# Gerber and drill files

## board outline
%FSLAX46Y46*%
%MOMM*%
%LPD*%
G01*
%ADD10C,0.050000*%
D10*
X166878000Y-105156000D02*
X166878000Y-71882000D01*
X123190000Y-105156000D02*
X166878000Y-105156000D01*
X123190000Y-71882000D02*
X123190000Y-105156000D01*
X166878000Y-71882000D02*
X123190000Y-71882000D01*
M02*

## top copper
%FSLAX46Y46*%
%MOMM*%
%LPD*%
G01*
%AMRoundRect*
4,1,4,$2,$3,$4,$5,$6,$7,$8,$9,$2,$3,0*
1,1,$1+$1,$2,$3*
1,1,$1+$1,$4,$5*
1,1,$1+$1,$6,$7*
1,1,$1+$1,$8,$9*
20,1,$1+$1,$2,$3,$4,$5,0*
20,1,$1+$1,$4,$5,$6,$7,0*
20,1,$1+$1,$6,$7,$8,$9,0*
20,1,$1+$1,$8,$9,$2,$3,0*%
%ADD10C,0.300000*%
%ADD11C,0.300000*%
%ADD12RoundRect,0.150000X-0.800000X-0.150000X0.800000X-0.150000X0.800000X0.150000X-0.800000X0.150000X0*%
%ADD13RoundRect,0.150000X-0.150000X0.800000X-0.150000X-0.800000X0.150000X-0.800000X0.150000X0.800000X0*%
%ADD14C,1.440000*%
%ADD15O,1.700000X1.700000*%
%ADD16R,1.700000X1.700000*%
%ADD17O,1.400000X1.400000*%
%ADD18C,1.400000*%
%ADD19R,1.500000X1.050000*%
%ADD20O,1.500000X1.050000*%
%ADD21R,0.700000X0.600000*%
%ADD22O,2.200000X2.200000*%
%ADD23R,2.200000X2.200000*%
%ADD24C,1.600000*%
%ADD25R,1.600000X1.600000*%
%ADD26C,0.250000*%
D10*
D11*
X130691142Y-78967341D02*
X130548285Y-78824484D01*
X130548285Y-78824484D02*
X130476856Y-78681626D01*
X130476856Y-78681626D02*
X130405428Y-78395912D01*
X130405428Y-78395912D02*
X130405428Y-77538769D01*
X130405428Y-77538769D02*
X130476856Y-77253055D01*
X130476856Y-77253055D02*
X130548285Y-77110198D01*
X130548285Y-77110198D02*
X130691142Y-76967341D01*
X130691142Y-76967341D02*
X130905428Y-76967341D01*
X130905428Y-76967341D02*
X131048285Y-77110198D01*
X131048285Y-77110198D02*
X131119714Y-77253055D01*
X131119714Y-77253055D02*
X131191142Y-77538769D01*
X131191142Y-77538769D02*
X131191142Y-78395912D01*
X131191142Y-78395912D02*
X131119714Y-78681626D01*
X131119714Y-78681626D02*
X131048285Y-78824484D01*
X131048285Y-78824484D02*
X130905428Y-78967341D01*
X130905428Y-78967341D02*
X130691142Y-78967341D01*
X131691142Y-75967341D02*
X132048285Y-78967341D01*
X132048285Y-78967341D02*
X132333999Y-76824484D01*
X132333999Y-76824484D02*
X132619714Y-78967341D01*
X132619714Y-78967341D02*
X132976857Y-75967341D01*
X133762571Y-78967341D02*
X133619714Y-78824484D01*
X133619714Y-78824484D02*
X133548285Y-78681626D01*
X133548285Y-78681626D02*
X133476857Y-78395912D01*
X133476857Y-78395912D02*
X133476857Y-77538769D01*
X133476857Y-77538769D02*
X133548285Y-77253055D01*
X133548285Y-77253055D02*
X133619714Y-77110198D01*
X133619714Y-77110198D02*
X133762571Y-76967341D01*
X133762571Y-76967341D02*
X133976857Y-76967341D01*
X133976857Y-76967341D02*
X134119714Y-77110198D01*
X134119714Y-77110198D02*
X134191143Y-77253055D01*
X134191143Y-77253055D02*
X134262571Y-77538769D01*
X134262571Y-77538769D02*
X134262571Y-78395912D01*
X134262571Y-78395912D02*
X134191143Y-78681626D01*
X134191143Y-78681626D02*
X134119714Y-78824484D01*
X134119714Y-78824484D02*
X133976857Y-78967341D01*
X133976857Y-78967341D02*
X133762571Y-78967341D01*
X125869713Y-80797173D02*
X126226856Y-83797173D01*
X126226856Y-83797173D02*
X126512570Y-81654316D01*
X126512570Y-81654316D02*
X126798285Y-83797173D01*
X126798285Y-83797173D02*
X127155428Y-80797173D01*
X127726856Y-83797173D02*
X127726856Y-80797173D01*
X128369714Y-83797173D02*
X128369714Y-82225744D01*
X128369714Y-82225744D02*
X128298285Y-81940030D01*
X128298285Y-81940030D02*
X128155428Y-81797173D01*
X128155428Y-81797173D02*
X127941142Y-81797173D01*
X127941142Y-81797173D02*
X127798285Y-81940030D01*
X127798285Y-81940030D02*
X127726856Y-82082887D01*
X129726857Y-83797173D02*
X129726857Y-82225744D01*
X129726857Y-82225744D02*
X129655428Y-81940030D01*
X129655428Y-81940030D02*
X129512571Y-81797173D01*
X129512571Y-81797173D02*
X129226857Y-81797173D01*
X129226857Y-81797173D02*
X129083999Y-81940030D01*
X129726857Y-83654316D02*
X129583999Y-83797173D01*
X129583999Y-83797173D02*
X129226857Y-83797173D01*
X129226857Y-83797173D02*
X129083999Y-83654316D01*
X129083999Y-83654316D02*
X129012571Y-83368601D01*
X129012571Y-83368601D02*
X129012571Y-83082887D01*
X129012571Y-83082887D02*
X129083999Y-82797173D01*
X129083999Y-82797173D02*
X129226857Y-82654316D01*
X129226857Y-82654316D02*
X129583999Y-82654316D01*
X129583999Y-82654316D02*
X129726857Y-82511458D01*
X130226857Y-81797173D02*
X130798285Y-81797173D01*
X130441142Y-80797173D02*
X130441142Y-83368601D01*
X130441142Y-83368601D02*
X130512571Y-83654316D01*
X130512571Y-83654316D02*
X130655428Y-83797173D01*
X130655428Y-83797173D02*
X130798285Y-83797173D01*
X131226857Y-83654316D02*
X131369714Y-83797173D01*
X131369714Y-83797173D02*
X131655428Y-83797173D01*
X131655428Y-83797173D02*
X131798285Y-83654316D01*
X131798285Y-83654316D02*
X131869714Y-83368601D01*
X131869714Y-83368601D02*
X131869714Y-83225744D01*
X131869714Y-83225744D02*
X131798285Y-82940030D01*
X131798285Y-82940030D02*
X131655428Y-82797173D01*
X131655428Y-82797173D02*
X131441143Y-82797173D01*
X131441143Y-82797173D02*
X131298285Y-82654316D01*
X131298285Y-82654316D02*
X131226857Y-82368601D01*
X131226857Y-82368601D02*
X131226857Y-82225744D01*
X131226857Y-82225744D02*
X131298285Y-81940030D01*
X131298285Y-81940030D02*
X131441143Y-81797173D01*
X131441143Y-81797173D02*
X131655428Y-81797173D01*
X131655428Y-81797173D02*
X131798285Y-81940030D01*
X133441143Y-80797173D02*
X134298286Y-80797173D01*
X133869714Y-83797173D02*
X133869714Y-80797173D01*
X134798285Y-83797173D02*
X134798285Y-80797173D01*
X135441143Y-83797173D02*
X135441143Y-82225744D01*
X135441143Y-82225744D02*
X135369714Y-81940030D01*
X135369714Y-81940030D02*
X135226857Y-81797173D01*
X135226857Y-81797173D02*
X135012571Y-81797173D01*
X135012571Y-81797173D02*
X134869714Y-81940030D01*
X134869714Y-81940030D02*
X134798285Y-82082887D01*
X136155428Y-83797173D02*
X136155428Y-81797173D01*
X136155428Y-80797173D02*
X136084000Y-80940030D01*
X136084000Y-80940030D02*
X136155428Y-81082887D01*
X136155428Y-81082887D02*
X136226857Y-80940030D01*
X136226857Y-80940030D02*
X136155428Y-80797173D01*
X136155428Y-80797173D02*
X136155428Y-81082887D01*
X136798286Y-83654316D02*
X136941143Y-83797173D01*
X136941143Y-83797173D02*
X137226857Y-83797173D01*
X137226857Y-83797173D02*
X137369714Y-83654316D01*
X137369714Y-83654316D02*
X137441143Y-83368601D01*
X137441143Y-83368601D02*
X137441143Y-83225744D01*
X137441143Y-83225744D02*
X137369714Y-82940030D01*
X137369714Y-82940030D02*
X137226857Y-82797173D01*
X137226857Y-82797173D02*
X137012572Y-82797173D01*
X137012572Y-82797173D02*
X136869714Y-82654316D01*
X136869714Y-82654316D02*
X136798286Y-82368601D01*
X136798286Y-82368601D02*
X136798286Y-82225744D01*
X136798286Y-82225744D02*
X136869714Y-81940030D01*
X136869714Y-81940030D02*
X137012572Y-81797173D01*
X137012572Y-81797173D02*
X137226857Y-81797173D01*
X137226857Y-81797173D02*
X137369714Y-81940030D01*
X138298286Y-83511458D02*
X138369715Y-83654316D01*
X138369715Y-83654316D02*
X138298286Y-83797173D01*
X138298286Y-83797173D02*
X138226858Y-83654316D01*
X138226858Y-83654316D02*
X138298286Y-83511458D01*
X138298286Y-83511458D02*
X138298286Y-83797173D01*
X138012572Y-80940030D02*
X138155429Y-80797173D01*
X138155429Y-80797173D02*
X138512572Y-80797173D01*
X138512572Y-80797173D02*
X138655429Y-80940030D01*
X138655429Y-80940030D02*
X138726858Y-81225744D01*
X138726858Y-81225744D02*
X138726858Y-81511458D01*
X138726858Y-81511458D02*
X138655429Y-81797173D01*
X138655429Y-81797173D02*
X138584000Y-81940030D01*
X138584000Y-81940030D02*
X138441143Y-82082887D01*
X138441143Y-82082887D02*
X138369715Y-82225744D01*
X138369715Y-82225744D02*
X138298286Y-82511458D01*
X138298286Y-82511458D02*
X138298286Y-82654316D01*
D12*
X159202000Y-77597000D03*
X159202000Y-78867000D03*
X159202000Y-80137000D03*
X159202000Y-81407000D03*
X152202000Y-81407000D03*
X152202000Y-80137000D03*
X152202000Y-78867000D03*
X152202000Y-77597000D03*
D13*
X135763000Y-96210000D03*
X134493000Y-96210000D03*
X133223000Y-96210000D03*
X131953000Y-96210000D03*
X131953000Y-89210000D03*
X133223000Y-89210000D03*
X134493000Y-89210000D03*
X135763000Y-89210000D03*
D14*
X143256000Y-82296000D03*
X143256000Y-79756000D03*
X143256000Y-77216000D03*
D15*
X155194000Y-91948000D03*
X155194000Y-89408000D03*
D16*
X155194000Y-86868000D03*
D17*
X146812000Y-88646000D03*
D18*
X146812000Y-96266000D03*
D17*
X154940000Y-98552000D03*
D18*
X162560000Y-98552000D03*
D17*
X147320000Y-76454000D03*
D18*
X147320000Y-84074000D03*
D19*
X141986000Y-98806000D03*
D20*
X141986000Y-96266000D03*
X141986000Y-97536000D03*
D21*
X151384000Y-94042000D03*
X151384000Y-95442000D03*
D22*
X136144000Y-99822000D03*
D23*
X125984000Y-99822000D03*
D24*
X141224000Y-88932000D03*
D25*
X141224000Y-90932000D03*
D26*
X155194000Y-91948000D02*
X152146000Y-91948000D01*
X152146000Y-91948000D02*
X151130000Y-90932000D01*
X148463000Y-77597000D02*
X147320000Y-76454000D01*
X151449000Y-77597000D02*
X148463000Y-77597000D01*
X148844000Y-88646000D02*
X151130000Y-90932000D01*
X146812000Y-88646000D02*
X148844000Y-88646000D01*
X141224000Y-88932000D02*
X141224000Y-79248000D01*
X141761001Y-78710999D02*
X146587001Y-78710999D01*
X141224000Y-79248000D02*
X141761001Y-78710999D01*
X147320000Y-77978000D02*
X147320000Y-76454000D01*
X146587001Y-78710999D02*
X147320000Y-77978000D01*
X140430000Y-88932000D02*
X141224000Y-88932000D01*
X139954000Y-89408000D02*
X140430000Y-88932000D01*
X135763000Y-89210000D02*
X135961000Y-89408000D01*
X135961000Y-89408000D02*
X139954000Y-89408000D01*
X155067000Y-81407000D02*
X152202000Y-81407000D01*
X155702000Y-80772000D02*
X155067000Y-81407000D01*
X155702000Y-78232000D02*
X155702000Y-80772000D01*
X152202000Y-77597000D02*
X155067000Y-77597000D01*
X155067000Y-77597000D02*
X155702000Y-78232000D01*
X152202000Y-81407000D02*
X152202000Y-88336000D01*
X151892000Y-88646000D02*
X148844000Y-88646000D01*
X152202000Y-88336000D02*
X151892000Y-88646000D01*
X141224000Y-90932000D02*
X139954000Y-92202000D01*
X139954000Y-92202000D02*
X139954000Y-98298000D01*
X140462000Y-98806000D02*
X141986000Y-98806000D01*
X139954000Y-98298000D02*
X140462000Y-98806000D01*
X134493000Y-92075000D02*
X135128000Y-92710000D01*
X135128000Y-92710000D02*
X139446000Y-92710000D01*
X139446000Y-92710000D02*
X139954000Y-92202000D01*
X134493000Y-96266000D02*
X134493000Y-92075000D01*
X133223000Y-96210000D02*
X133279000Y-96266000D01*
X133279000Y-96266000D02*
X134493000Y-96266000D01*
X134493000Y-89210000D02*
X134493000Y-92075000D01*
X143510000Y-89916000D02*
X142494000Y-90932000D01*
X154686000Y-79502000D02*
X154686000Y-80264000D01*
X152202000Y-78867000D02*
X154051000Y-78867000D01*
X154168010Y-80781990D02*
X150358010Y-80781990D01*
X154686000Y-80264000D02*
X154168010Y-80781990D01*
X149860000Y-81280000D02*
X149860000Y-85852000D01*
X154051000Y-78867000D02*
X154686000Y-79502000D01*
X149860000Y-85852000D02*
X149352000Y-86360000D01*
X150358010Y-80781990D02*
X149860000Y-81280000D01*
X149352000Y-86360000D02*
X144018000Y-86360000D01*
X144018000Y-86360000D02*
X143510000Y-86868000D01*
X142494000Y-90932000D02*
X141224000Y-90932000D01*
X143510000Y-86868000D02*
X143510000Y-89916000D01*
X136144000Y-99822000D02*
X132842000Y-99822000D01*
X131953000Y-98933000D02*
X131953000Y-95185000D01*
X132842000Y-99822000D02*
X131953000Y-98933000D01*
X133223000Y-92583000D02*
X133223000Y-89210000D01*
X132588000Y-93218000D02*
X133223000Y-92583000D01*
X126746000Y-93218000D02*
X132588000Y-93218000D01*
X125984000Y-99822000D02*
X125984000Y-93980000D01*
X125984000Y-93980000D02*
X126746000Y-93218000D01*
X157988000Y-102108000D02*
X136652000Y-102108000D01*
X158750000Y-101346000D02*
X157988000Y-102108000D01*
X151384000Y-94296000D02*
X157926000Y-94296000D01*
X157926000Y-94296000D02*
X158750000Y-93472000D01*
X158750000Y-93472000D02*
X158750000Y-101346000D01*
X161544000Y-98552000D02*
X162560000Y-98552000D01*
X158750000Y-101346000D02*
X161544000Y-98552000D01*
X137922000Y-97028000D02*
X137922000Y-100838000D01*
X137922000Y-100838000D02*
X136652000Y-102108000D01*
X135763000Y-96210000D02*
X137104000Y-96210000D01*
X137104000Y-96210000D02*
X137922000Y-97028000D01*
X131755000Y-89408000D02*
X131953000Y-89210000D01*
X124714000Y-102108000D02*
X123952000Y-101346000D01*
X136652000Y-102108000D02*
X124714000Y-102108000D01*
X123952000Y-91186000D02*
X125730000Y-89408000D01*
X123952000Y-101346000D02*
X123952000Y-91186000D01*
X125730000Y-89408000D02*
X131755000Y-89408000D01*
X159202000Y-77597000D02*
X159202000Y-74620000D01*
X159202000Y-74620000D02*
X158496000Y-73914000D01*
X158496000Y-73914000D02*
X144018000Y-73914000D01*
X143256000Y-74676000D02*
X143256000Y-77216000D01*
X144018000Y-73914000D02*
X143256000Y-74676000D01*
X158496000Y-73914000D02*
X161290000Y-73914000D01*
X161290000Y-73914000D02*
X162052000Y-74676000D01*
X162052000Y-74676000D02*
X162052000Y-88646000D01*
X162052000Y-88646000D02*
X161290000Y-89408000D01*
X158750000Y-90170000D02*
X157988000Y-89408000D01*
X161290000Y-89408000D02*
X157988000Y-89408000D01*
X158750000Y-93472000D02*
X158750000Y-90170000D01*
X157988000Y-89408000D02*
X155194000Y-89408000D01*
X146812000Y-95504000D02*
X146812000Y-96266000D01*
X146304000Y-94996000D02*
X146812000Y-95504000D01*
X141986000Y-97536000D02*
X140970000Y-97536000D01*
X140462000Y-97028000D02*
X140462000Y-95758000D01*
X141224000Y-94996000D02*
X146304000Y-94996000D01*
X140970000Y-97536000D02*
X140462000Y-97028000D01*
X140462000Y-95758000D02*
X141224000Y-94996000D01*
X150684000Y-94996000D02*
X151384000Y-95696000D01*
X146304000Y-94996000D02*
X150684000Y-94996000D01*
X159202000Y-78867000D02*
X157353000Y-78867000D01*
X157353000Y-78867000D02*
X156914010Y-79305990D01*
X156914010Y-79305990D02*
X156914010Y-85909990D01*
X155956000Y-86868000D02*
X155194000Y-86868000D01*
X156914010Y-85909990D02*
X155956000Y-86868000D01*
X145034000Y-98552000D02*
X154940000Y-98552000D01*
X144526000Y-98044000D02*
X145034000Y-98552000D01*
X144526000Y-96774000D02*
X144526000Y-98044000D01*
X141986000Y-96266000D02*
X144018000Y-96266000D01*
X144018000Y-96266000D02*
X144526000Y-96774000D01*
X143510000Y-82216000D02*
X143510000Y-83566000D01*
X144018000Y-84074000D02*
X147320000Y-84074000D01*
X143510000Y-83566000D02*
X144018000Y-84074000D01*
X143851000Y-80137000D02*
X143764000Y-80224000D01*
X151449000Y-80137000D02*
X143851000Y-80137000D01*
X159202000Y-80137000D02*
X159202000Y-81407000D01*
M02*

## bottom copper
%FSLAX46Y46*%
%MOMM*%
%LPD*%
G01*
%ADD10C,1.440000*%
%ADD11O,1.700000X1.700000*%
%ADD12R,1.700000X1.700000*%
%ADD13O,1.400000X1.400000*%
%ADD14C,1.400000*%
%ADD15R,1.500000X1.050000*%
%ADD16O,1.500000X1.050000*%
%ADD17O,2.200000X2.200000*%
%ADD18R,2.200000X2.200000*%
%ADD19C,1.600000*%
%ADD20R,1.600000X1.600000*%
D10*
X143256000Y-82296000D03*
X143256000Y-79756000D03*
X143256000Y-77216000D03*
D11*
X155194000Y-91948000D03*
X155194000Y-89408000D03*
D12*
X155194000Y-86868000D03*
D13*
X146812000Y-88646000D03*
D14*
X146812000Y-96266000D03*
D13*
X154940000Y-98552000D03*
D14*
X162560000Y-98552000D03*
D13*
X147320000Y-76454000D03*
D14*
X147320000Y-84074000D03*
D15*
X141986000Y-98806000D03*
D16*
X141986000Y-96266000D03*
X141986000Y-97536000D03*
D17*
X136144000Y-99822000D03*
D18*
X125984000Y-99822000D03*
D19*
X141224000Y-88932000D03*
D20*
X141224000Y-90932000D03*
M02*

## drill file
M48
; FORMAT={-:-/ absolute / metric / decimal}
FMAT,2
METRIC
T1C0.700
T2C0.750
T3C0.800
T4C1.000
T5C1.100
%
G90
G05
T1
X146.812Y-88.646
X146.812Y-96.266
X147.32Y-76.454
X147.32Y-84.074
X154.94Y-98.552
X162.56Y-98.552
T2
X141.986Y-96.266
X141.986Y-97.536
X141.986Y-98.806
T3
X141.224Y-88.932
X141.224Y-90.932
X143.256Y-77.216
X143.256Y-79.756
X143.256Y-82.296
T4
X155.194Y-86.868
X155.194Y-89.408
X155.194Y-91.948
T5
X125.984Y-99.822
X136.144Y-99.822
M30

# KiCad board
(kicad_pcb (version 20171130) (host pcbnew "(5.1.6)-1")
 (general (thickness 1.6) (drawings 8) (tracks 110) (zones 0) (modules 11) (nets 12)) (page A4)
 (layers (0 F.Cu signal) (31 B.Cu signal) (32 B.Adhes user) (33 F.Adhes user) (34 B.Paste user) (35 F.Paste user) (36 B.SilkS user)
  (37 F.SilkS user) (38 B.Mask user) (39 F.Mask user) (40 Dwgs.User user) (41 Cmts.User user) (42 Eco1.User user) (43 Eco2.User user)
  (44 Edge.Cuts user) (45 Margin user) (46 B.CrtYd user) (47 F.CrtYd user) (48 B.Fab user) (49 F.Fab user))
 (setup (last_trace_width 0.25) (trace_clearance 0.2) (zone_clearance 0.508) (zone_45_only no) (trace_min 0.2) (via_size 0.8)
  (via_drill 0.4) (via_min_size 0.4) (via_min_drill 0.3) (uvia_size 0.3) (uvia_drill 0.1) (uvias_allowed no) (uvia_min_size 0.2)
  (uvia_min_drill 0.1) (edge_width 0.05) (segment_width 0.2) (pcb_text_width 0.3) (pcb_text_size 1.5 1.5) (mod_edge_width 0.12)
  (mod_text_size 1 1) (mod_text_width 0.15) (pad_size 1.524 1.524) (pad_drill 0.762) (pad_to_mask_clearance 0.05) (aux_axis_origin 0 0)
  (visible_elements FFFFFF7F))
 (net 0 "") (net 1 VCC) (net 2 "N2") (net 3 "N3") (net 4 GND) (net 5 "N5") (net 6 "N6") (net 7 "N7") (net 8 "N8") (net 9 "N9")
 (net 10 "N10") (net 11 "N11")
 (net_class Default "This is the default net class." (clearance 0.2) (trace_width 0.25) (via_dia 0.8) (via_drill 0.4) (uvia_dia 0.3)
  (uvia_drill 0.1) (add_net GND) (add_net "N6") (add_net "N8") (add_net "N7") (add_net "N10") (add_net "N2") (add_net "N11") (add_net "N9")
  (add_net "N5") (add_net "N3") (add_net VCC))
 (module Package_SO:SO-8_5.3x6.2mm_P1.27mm (layer F.Cu) (at 155.702 79.502)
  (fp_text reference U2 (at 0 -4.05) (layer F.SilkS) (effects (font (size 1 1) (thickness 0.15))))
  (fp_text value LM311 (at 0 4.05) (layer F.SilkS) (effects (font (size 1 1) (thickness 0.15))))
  (pad 8 smd roundrect (at 3.5 -1.905) (size 1.9 0.6) (layers F.Cu F.Paste F.Mask) (roundrect_rratio 0.25) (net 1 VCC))
  (pad 7 smd roundrect (at 3.5 -0.635) (size 1.9 0.6) (layers F.Cu F.Paste F.Mask) (roundrect_rratio 0.25) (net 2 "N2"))
  (pad 6 smd roundrect (at 3.5 0.635) (size 1.9 0.6) (layers F.Cu F.Paste F.Mask) (roundrect_rratio 0.25) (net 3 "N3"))
  (pad 5 smd roundrect (at 3.5 1.905) (size 1.9 0.6) (layers F.Cu F.Paste F.Mask) (roundrect_rratio 0.25) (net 3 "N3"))
  (pad 4 smd roundrect (at -3.5 1.905) (size 1.9 0.6) (layers F.Cu F.Paste F.Mask) (roundrect_rratio 0.25) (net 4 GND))
  (pad 3 smd roundrect (at -3.5 0.635) (size 1.9 0.6) (layers F.Cu F.Paste F.Mask) (roundrect_rratio 0.25) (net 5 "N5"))
  (pad 2 smd roundrect (at -3.5 -0.635) (size 1.9 0.6) (layers F.Cu F.Paste F.Mask) (roundrect_rratio 0.25) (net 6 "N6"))
  (pad 1 smd roundrect (at -3.5 -1.905) (size 1.9 0.6) (layers F.Cu F.Paste F.Mask) (roundrect_rratio 0.25) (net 4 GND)))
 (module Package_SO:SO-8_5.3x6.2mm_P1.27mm (layer F.Cu) (at 133.858 92.71 270)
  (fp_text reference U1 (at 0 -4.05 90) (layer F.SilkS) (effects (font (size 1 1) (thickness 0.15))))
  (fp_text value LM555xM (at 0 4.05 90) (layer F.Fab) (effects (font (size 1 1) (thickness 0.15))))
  (pad 8 smd roundrect (at 3.5 -1.905 270) (size 1.9 0.6) (layers F.Cu F.Paste F.Mask) (roundrect_rratio 0.25) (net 1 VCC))
  (pad 7 smd roundrect (at 3.5 -0.635 270) (size 1.9 0.6) (layers F.Cu F.Paste F.Mask) (roundrect_rratio 0.25) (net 6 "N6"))
  (pad 6 smd roundrect (at 3.5 0.635 270) (size 1.9 0.6) (layers F.Cu F.Paste F.Mask) (roundrect_rratio 0.25) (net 6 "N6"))
  (pad 5 smd roundrect (at 3.5 1.905 270) (size 1.9 0.6) (layers F.Cu F.Paste F.Mask) (roundrect_rratio 0.25) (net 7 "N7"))
  (pad 4 smd roundrect (at -3.5 1.905 270) (size 1.9 0.6) (layers F.Cu F.Paste F.Mask) (roundrect_rratio 0.25) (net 1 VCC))
  (pad 3 smd roundrect (at -3.5 0.635 270) (size 1.9 0.6) (layers F.Cu F.Paste F.Mask) (roundrect_rratio 0.25) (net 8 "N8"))
  (pad 2 smd roundrect (at -3.5 -0.635 270) (size 1.9 0.6) (layers F.Cu F.Paste F.Mask) (roundrect_rratio 0.25) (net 6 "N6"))
  (pad 1 smd roundrect (at -3.5 -1.905 270) (size 1.9 0.6) (layers F.Cu F.Paste F.Mask) (roundrect_rratio 0.25) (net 4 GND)))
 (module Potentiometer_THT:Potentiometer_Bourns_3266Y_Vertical (layer F.Cu) (at 143.256 77.216 90)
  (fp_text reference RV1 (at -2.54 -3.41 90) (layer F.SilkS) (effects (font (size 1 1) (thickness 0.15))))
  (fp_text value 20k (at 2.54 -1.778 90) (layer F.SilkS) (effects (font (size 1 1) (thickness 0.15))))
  (pad 3 thru_hole circle (at -5.08 0 90) (size 1.44 1.44) (drill 0.8) (layers *.Cu *.Mask) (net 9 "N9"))
  (pad 2 thru_hole circle (at -2.54 0 90) (size 1.44 1.44) (drill 0.8) (layers *.Cu *.Mask) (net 5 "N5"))
  (pad 1 thru_hole circle (at 0 0 90) (size 1.44 1.44) (drill 0.8) (layers *.Cu *.Mask) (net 1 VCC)))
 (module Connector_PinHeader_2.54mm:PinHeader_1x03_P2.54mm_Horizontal (layer F.Cu) (at 155.194 86.868)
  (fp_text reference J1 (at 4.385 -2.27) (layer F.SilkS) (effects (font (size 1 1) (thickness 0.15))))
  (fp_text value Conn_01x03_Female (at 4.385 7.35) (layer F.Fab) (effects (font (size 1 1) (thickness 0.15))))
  (pad 3 thru_hole oval (at 0 5.08) (size 1.7 1.7) (drill 1) (layers *.Cu *.Mask) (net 4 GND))
  (pad 2 thru_hole oval (at 0 2.54) (size 1.7 1.7) (drill 1) (layers *.Cu *.Mask) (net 1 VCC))
  (pad 1 thru_hole rect (at 0 0) (size 1.7 1.7) (drill 1) (layers *.Cu *.Mask) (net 2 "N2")))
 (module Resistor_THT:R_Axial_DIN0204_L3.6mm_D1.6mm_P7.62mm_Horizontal (layer F.Cu) (at 146.812 96.266 90)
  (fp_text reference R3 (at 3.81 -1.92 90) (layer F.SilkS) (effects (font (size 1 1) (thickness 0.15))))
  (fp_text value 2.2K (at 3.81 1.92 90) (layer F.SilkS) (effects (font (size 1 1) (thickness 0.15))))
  (pad 2 thru_hole oval (at 7.62 0 90) (size 1.4 1.4) (drill 0.7) (layers *.Cu *.Mask) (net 4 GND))
  (pad 1 thru_hole circle (at 0 0 90) (size 1.4 1.4) (drill 0.7) (layers *.Cu *.Mask) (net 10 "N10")))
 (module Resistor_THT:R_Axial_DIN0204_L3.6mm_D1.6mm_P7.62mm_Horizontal (layer F.Cu) (at 162.56 98.552 180)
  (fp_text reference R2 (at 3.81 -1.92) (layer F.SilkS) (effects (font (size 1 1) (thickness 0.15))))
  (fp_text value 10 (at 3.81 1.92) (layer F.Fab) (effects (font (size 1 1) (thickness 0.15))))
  (pad 2 thru_hole oval (at 7.62 0 180) (size 1.4 1.4) (drill 0.7) (layers *.Cu *.Mask) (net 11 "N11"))
  (pad 1 thru_hole circle (at 0 0 180) (size 1.4 1.4) (drill 0.7) (layers *.Cu *.Mask) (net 1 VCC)))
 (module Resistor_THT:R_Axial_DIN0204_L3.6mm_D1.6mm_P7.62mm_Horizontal (layer F.Cu) (at 147.32 84.074 90)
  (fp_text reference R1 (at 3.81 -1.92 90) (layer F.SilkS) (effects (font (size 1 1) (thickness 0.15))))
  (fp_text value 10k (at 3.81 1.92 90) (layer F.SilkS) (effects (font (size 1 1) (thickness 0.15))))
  (pad 2 thru_hole oval (at 7.62 0 90) (size 1.4 1.4) (drill 0.7) (layers *.Cu *.Mask) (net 4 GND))
  (pad 1 thru_hole circle (at 0 0 90) (size 1.4 1.4) (drill 0.7) (layers *.Cu *.Mask) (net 9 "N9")))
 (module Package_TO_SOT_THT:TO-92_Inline (layer F.Cu) (at 141.986 98.806 90)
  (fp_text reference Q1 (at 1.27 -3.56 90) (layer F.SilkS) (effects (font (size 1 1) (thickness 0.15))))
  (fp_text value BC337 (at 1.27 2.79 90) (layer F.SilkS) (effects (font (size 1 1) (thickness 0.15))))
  (pad 1 thru_hole rect (at 0 0 90) (size 1.05 1.5) (drill 0.75) (layers *.Cu *.Mask) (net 6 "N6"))
  (pad 3 thru_hole oval (at 2.54 0 90) (size 1.05 1.5) (drill 0.75) (layers *.Cu *.Mask) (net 11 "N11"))
  (pad 2 thru_hole oval (at 1.27 0 90) (size 1.05 1.5) (drill 0.75) (layers *.Cu *.Mask) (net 10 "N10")))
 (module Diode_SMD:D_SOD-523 (layer F.Cu) (at 151.384 94.742 270)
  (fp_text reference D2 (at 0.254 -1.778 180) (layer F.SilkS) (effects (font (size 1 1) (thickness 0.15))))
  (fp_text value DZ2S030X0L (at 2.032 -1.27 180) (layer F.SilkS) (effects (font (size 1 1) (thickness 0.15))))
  (pad 1 smd rect (at -0.7 0 90) (size 0.6 0.7) (layers F.Cu F.Paste F.Mask) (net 1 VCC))
  (pad 2 smd rect (at 0.7 0 90) (size 0.6 0.7) (layers F.Cu F.Paste F.Mask) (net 10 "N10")))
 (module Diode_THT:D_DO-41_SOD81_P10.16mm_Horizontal (layer F.Cu) (at 125.984 99.822)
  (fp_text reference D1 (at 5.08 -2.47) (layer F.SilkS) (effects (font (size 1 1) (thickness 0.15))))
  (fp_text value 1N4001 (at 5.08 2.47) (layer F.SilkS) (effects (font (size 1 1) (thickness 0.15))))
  (pad 2 thru_hole oval (at 10.16 0) (size 2.2 2.2) (drill 1.1) (layers *.Cu *.Mask) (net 7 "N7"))
  (pad 1 thru_hole rect (at 0 0) (size 2.2 2.2) (drill 1.1) (layers *.Cu *.Mask) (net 8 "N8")))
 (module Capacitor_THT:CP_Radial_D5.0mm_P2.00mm (layer F.Cu) (at 141.224 90.932 90)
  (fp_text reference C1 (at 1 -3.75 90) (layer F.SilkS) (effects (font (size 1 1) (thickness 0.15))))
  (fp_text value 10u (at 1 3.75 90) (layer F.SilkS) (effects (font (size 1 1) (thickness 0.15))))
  (pad 2 thru_hole circle (at 2 0 90) (size 1.6 1.6) (drill 0.8) (layers *.Cu *.Mask) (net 4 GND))
  (pad 1 thru_hole rect (at 0 0 90) (size 1.6 1.6) (drill 0.8) (layers *.Cu *.Mask) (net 6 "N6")))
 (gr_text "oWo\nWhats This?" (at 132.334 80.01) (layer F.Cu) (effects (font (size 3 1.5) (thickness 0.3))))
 (gr_line (start 166.878 105.156) (end 166.878 71.882) (layer Edge.Cuts) (width 0.05))
 (gr_line (start 123.19 105.156) (end 166.878 105.156) (layer Edge.Cuts) (width 0.05))
 (gr_line (start 123.19 71.882) (end 123.19 105.156) (layer Edge.Cuts) (width 0.05))
 (gr_line (start 166.878 71.882) (end 123.19 71.882) (layer Edge.Cuts) (width 0.05))
 (segment (start 155.194 91.948) (end 152.146 91.948) (width 0.25) (layer F.Cu) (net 4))
 (segment (start 152.146 91.948) (end 151.13 90.932) (width 0.25) (layer F.Cu) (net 4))
 (segment (start 148.463 77.597) (end 147.32 76.454) (width 0.25) (layer F.Cu) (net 4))
 (segment (start 151.449 77.597) (end 148.463 77.597) (width 0.25) (layer F.Cu) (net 4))
 (segment (start 148.844 88.646) (end 151.13 90.932) (width 0.25) (layer F.Cu) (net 4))
 (segment (start 146.812 88.646) (end 148.844 88.646) (width 0.25) (layer F.Cu) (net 4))
 (segment (start 141.224 88.932) (end 141.224 79.248) (width 0.25) (layer F.Cu) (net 4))
 (segment (start 141.761001 78.710999) (end 146.587001 78.710999) (width 0.25) (layer F.Cu) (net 4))
 (segment (start 141.224 79.248) (end 141.761001 78.710999) (width 0.25) (layer F.Cu) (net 4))
 (segment (start 147.32 77.978) (end 147.32 76.454) (width 0.25) (layer F.Cu) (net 4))
 (segment (start 146.587001 78.710999) (end 147.32 77.978) (width 0.25) (layer F.Cu) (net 4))
 (segment (start 140.43 88.932) (end 141.224 88.932) (width 0.25) (layer F.Cu) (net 4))
 (segment (start 139.954 89.408) (end 140.43 88.932) (width 0.25) (layer F.Cu) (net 4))
 (segment (start 135.763 89.21) (end 135.961 89.408) (width 0.25) (layer F.Cu) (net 4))
 (segment (start 135.961 89.408) (end 139.954 89.408) (width 0.25) (layer F.Cu) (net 4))
 (segment (start 155.067 81.407) (end 152.202 81.407) (width 0.25) (layer F.Cu) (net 4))
 (segment (start 155.702 80.772) (end 155.067 81.407) (width 0.25) (layer F.Cu) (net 4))
 (segment (start 155.702 78.232) (end 155.702 80.772) (width 0.25) (layer F.Cu) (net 4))
 (segment (start 152.202 77.597) (end 155.067 77.597) (width 0.25) (layer F.Cu) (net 4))
 (segment (start 155.067 77.597) (end 155.702 78.232) (width 0.25) (layer F.Cu) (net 4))
 (segment (start 152.202 81.407) (end 152.202 88.336) (width 0.25) (layer F.Cu) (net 4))
 (segment (start 151.892 88.646) (end 148.844 88.646) (width 0.25) (layer F.Cu) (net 4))
 (segment (start 152.202 88.336) (end 151.892 88.646) (width 0.25) (layer F.Cu) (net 4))
 (segment (start 141.224 90.932) (end 139.954 92.202) (width 0.25) (layer F.Cu) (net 6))
 (segment (start 139.954 92.202) (end 139.954 98.298) (width 0.25) (layer F.Cu) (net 6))
 (segment (start 140.462 98.806) (end 141.986 98.806) (width 0.25) (layer F.Cu) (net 6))
 (segment (start 139.954 98.298) (end 140.462 98.806) (width 0.25) (layer F.Cu) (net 6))
 (segment (start 134.493 92.075) (end 135.128 92.71) (width 0.25) (layer F.Cu) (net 6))
 (segment (start 135.128 92.71) (end 139.446 92.71) (width 0.25) (layer F.Cu) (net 6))
 (segment (start 139.446 92.71) (end 139.954 92.202) (width 0.25) (layer F.Cu) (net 6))
 (segment (start 134.493 96.266) (end 134.493 92.075) (width 0.25) (layer F.Cu) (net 6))
 (segment (start 133.223 96.21) (end 133.279 96.266) (width 0.25) (layer F.Cu) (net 6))
 (segment (start 133.279 96.266) (end 134.493 96.266) (width 0.25) (layer F.Cu) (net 6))
 (segment (start 134.493 89.21) (end 134.493 92.075) (width 0.25) (layer F.Cu) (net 6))
 (segment (start 143.51 89.916) (end 142.494 90.932) (width 0.25) (layer F.Cu) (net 6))
 (segment (start 154.686 79.502) (end 154.686 80.264) (width 0.25) (layer F.Cu) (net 6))
 (segment (start 152.202 78.867) (end 154.051 78.867) (width 0.25) (layer F.Cu) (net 6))
 (segment (start 154.16801 80.78199) (end 150.35801 80.78199) (width 0.25) (layer F.Cu) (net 6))
 (segment (start 154.686 80.264) (end 154.16801 80.78199) (width 0.25) (layer F.Cu) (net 6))
 (segment (start 149.86 81.28) (end 149.86 85.852) (width 0.25) (layer F.Cu) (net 6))
 (segment (start 154.051 78.867) (end 154.686 79.502) (width 0.25) (layer F.Cu) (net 6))
 (segment (start 149.86 85.852) (end 149.352 86.36) (width 0.25) (layer F.Cu) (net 6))
 (segment (start 150.35801 80.78199) (end 149.86 81.28) (width 0.25) (layer F.Cu) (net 6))
 (segment (start 149.352 86.36) (end 144.018 86.36) (width 0.25) (layer F.Cu) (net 6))
 (segment (start 144.018 86.36) (end 143.51 86.868) (width 0.25) (layer F.Cu) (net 6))
 (segment (start 142.494 90.932) (end 141.224 90.932) (width 0.25) (layer F.Cu) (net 6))
 (segment (start 143.51 86.868) (end 143.51 89.916) (width 0.25) (layer F.Cu) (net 6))
 (segment (start 136.144 99.822) (end 132.842 99.822) (width 0.25) (layer F.Cu) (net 7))
 (segment (start 131.953 98.933) (end 131.953 95.185) (width 0.25) (layer F.Cu) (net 7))
 (segment (start 132.842 99.822) (end 131.953 98.933) (width 0.25) (layer F.Cu) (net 7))
 (segment (start 133.223 92.583) (end 133.223 89.21) (width 0.25) (layer F.Cu) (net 8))
 (segment (start 132.588 93.218) (end 133.223 92.583) (width 0.25) (layer F.Cu) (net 8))
 (segment (start 126.746 93.218) (end 132.588 93.218) (width 0.25) (layer F.Cu) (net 8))
 (segment (start 125.984 99.822) (end 125.984 93.98) (width 0.25) (layer F.Cu) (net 8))
 (segment (start 125.984 93.98) (end 126.746 93.218) (width 0.25) (layer F.Cu) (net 8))
 (segment (start 157.988 102.108) (end 136.652 102.108) (width 0.25) (layer F.Cu) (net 1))
 (segment (start 158.75 101.346) (end 157.988 102.108) (width 0.25) (layer F.Cu) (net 1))
 (segment (start 151.384 94.296) (end 157.926 94.296) (width 0.25) (layer F.Cu) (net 1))
 (segment (start 157.926 94.296) (end 158.75 93.472) (width 0.25) (layer F.Cu) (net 1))
 (segment (start 158.75 93.472) (end 158.75 101.346) (width 0.25) (layer F.Cu) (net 1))
 (segment (start 161.544 98.552) (end 162.56 98.552) (width 0.25) (layer F.Cu) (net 1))
 (segment (start 158.75 101.346) (end 161.544 98.552) (width 0.25) (layer F.Cu) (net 1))
 (segment (start 137.922 97.028) (end 137.922 100.838) (width 0.25) (layer F.Cu) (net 1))
 (segment (start 137.922 100.838) (end 136.652 102.108) (width 0.25) (layer F.Cu) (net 1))
 (segment (start 135.763 96.21) (end 137.104 96.21) (width 0.25) (layer F.Cu) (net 1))
 (segment (start 137.104 96.21) (end 137.922 97.028) (width 0.25) (layer F.Cu) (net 1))
 (segment (start 131.755 89.408) (end 131.953 89.21) (width 0.25) (layer F.Cu) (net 1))
 (segment (start 124.714 102.108) (end 123.952 101.346) (width 0.25) (layer F.Cu) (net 1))
 (segment (start 136.652 102.108) (end 124.714 102.108) (width 0.25) (layer F.Cu) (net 1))
 (segment (start 123.952 91.186) (end 125.73 89.408) (width 0.25) (layer F.Cu) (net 1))
 (segment (start 123.952 101.346) (end 123.952 91.186) (width 0.25) (layer F.Cu) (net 1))
 (segment (start 125.73 89.408) (end 131.755 89.408) (width 0.25) (layer F.Cu) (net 1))
 (segment (start 159.202 77.597) (end 159.202 74.62) (width 0.25) (layer F.Cu) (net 1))
 (segment (start 159.202 74.62) (end 158.496 73.914) (width 0.25) (layer F.Cu) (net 1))
 (segment (start 158.496 73.914) (end 144.018 73.914) (width 0.25) (layer F.Cu) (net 1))
 (segment (start 143.256 74.676) (end 143.256 77.216) (width 0.25) (layer F.Cu) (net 1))
 (segment (start 144.018 73.914) (end 143.256 74.676) (width 0.25) (layer F.Cu) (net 1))
 (segment (start 158.496 73.914) (end 161.29 73.914) (width 0.25) (layer F.Cu) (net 1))
 (segment (start 161.29 73.914) (end 162.052 74.676) (width 0.25) (layer F.Cu) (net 1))
 (segment (start 162.052 74.676) (end 162.052 88.646) (width 0.25) (layer F.Cu) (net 1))
 (segment (start 162.052 88.646) (end 161.29 89.408) (width 0.25) (layer F.Cu) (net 1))
 (segment (start 158.75 90.17) (end 157.988 89.408) (width 0.25) (layer F.Cu) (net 1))
 (segment (start 161.29 89.408) (end 157.988 89.408) (width 0.25) (layer F.Cu) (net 1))
 (segment (start 158.75 93.472) (end 158.75 90.17) (width 0.25) (layer F.Cu) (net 1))
 (segment (start 157.988 89.408) (end 155.194 89.408) (width 0.25) (layer F.Cu) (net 1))
 (segment (start 146.812 95.504) (end 146.812 96.266) (width 0.25) (layer F.Cu) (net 10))
 (segment (start 146.304 94.996) (end 146.812 95.504) (width 0.25) (layer F.Cu) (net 10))
 (segment (start 141.986 97.536) (end 140.97 97.536) (width 0.25) (layer F.Cu) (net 10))
 (segment (start 140.462 97.028) (end 140.462 95.758) (width 0.25) (layer F.Cu) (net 10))
 (segment (start 141.224 94.996) (end 146.304 94.996) (width 0.25) (layer F.Cu) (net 10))
 (segment (start 140.97 97.536) (end 140.462 97.028) (width 0.25) (layer F.Cu) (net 10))
 (segment (start 140.462 95.758) (end 141.224 94.996) (width 0.25) (layer F.Cu) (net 10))
 (segment (start 150.684 94.996) (end 151.384 95.696) (width 0.25) (layer F.Cu) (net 10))
 (segment (start 146.304 94.996) (end 150.684 94.996) (width 0.25) (layer F.Cu) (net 10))
 (segment (start 159.202 78.867) (end 157.353 78.867) (width 0.25) (layer F.Cu) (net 2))
 (segment (start 157.353 78.867) (end 156.91401 79.30599) (width 0.25) (layer F.Cu) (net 2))
 (segment (start 156.91401 79.30599) (end 156.91401 85.90999) (width 0.25) (layer F.Cu) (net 2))
 (segment (start 155.956 86.868) (end 155.194 86.868) (width 0.25) (layer F.Cu) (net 2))
 (segment (start 156.91401 85.90999) (end 155.956 86.868) (width 0.25) (layer F.Cu) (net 2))
 (segment (start 145.034 98.552) (end 154.94 98.552) (width 0.25) (layer F.Cu) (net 11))
 (segment (start 144.526 98.044) (end 145.034 98.552) (width 0.25) (layer F.Cu) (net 11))
 (segment (start 144.526 96.774) (end 144.526 98.044) (width 0.25) (layer F.Cu) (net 11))
 (segment (start 141.986 96.266) (end 144.018 96.266) (width 0.25) (layer F.Cu) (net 11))
 (segment (start 144.018 96.266) (end 144.526 96.774) (width 0.25) (layer F.Cu) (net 11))
 (segment (start 143.51 82.216) (end 143.51 83.566) (width 0.25) (layer F.Cu) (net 9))
 (segment (start 144.018 84.074) (end 147.32 84.074) (width 0.25) (layer F.Cu) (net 9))
 (segment (start 143.51 83.566) (end 144.018 84.074) (width 0.25) (layer F.Cu) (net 9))
 (segment (start 143.851 80.137) (end 143.764 80.224) (width 0.25) (layer F.Cu) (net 5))
 (segment (start 151.449 80.137) (end 143.851 80.137) (width 0.25) (layer F.Cu) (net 5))
 (segment (start 159.202 80.137) (end 159.202 81.407) (width 0.25) (layer F.Cu) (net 3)))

